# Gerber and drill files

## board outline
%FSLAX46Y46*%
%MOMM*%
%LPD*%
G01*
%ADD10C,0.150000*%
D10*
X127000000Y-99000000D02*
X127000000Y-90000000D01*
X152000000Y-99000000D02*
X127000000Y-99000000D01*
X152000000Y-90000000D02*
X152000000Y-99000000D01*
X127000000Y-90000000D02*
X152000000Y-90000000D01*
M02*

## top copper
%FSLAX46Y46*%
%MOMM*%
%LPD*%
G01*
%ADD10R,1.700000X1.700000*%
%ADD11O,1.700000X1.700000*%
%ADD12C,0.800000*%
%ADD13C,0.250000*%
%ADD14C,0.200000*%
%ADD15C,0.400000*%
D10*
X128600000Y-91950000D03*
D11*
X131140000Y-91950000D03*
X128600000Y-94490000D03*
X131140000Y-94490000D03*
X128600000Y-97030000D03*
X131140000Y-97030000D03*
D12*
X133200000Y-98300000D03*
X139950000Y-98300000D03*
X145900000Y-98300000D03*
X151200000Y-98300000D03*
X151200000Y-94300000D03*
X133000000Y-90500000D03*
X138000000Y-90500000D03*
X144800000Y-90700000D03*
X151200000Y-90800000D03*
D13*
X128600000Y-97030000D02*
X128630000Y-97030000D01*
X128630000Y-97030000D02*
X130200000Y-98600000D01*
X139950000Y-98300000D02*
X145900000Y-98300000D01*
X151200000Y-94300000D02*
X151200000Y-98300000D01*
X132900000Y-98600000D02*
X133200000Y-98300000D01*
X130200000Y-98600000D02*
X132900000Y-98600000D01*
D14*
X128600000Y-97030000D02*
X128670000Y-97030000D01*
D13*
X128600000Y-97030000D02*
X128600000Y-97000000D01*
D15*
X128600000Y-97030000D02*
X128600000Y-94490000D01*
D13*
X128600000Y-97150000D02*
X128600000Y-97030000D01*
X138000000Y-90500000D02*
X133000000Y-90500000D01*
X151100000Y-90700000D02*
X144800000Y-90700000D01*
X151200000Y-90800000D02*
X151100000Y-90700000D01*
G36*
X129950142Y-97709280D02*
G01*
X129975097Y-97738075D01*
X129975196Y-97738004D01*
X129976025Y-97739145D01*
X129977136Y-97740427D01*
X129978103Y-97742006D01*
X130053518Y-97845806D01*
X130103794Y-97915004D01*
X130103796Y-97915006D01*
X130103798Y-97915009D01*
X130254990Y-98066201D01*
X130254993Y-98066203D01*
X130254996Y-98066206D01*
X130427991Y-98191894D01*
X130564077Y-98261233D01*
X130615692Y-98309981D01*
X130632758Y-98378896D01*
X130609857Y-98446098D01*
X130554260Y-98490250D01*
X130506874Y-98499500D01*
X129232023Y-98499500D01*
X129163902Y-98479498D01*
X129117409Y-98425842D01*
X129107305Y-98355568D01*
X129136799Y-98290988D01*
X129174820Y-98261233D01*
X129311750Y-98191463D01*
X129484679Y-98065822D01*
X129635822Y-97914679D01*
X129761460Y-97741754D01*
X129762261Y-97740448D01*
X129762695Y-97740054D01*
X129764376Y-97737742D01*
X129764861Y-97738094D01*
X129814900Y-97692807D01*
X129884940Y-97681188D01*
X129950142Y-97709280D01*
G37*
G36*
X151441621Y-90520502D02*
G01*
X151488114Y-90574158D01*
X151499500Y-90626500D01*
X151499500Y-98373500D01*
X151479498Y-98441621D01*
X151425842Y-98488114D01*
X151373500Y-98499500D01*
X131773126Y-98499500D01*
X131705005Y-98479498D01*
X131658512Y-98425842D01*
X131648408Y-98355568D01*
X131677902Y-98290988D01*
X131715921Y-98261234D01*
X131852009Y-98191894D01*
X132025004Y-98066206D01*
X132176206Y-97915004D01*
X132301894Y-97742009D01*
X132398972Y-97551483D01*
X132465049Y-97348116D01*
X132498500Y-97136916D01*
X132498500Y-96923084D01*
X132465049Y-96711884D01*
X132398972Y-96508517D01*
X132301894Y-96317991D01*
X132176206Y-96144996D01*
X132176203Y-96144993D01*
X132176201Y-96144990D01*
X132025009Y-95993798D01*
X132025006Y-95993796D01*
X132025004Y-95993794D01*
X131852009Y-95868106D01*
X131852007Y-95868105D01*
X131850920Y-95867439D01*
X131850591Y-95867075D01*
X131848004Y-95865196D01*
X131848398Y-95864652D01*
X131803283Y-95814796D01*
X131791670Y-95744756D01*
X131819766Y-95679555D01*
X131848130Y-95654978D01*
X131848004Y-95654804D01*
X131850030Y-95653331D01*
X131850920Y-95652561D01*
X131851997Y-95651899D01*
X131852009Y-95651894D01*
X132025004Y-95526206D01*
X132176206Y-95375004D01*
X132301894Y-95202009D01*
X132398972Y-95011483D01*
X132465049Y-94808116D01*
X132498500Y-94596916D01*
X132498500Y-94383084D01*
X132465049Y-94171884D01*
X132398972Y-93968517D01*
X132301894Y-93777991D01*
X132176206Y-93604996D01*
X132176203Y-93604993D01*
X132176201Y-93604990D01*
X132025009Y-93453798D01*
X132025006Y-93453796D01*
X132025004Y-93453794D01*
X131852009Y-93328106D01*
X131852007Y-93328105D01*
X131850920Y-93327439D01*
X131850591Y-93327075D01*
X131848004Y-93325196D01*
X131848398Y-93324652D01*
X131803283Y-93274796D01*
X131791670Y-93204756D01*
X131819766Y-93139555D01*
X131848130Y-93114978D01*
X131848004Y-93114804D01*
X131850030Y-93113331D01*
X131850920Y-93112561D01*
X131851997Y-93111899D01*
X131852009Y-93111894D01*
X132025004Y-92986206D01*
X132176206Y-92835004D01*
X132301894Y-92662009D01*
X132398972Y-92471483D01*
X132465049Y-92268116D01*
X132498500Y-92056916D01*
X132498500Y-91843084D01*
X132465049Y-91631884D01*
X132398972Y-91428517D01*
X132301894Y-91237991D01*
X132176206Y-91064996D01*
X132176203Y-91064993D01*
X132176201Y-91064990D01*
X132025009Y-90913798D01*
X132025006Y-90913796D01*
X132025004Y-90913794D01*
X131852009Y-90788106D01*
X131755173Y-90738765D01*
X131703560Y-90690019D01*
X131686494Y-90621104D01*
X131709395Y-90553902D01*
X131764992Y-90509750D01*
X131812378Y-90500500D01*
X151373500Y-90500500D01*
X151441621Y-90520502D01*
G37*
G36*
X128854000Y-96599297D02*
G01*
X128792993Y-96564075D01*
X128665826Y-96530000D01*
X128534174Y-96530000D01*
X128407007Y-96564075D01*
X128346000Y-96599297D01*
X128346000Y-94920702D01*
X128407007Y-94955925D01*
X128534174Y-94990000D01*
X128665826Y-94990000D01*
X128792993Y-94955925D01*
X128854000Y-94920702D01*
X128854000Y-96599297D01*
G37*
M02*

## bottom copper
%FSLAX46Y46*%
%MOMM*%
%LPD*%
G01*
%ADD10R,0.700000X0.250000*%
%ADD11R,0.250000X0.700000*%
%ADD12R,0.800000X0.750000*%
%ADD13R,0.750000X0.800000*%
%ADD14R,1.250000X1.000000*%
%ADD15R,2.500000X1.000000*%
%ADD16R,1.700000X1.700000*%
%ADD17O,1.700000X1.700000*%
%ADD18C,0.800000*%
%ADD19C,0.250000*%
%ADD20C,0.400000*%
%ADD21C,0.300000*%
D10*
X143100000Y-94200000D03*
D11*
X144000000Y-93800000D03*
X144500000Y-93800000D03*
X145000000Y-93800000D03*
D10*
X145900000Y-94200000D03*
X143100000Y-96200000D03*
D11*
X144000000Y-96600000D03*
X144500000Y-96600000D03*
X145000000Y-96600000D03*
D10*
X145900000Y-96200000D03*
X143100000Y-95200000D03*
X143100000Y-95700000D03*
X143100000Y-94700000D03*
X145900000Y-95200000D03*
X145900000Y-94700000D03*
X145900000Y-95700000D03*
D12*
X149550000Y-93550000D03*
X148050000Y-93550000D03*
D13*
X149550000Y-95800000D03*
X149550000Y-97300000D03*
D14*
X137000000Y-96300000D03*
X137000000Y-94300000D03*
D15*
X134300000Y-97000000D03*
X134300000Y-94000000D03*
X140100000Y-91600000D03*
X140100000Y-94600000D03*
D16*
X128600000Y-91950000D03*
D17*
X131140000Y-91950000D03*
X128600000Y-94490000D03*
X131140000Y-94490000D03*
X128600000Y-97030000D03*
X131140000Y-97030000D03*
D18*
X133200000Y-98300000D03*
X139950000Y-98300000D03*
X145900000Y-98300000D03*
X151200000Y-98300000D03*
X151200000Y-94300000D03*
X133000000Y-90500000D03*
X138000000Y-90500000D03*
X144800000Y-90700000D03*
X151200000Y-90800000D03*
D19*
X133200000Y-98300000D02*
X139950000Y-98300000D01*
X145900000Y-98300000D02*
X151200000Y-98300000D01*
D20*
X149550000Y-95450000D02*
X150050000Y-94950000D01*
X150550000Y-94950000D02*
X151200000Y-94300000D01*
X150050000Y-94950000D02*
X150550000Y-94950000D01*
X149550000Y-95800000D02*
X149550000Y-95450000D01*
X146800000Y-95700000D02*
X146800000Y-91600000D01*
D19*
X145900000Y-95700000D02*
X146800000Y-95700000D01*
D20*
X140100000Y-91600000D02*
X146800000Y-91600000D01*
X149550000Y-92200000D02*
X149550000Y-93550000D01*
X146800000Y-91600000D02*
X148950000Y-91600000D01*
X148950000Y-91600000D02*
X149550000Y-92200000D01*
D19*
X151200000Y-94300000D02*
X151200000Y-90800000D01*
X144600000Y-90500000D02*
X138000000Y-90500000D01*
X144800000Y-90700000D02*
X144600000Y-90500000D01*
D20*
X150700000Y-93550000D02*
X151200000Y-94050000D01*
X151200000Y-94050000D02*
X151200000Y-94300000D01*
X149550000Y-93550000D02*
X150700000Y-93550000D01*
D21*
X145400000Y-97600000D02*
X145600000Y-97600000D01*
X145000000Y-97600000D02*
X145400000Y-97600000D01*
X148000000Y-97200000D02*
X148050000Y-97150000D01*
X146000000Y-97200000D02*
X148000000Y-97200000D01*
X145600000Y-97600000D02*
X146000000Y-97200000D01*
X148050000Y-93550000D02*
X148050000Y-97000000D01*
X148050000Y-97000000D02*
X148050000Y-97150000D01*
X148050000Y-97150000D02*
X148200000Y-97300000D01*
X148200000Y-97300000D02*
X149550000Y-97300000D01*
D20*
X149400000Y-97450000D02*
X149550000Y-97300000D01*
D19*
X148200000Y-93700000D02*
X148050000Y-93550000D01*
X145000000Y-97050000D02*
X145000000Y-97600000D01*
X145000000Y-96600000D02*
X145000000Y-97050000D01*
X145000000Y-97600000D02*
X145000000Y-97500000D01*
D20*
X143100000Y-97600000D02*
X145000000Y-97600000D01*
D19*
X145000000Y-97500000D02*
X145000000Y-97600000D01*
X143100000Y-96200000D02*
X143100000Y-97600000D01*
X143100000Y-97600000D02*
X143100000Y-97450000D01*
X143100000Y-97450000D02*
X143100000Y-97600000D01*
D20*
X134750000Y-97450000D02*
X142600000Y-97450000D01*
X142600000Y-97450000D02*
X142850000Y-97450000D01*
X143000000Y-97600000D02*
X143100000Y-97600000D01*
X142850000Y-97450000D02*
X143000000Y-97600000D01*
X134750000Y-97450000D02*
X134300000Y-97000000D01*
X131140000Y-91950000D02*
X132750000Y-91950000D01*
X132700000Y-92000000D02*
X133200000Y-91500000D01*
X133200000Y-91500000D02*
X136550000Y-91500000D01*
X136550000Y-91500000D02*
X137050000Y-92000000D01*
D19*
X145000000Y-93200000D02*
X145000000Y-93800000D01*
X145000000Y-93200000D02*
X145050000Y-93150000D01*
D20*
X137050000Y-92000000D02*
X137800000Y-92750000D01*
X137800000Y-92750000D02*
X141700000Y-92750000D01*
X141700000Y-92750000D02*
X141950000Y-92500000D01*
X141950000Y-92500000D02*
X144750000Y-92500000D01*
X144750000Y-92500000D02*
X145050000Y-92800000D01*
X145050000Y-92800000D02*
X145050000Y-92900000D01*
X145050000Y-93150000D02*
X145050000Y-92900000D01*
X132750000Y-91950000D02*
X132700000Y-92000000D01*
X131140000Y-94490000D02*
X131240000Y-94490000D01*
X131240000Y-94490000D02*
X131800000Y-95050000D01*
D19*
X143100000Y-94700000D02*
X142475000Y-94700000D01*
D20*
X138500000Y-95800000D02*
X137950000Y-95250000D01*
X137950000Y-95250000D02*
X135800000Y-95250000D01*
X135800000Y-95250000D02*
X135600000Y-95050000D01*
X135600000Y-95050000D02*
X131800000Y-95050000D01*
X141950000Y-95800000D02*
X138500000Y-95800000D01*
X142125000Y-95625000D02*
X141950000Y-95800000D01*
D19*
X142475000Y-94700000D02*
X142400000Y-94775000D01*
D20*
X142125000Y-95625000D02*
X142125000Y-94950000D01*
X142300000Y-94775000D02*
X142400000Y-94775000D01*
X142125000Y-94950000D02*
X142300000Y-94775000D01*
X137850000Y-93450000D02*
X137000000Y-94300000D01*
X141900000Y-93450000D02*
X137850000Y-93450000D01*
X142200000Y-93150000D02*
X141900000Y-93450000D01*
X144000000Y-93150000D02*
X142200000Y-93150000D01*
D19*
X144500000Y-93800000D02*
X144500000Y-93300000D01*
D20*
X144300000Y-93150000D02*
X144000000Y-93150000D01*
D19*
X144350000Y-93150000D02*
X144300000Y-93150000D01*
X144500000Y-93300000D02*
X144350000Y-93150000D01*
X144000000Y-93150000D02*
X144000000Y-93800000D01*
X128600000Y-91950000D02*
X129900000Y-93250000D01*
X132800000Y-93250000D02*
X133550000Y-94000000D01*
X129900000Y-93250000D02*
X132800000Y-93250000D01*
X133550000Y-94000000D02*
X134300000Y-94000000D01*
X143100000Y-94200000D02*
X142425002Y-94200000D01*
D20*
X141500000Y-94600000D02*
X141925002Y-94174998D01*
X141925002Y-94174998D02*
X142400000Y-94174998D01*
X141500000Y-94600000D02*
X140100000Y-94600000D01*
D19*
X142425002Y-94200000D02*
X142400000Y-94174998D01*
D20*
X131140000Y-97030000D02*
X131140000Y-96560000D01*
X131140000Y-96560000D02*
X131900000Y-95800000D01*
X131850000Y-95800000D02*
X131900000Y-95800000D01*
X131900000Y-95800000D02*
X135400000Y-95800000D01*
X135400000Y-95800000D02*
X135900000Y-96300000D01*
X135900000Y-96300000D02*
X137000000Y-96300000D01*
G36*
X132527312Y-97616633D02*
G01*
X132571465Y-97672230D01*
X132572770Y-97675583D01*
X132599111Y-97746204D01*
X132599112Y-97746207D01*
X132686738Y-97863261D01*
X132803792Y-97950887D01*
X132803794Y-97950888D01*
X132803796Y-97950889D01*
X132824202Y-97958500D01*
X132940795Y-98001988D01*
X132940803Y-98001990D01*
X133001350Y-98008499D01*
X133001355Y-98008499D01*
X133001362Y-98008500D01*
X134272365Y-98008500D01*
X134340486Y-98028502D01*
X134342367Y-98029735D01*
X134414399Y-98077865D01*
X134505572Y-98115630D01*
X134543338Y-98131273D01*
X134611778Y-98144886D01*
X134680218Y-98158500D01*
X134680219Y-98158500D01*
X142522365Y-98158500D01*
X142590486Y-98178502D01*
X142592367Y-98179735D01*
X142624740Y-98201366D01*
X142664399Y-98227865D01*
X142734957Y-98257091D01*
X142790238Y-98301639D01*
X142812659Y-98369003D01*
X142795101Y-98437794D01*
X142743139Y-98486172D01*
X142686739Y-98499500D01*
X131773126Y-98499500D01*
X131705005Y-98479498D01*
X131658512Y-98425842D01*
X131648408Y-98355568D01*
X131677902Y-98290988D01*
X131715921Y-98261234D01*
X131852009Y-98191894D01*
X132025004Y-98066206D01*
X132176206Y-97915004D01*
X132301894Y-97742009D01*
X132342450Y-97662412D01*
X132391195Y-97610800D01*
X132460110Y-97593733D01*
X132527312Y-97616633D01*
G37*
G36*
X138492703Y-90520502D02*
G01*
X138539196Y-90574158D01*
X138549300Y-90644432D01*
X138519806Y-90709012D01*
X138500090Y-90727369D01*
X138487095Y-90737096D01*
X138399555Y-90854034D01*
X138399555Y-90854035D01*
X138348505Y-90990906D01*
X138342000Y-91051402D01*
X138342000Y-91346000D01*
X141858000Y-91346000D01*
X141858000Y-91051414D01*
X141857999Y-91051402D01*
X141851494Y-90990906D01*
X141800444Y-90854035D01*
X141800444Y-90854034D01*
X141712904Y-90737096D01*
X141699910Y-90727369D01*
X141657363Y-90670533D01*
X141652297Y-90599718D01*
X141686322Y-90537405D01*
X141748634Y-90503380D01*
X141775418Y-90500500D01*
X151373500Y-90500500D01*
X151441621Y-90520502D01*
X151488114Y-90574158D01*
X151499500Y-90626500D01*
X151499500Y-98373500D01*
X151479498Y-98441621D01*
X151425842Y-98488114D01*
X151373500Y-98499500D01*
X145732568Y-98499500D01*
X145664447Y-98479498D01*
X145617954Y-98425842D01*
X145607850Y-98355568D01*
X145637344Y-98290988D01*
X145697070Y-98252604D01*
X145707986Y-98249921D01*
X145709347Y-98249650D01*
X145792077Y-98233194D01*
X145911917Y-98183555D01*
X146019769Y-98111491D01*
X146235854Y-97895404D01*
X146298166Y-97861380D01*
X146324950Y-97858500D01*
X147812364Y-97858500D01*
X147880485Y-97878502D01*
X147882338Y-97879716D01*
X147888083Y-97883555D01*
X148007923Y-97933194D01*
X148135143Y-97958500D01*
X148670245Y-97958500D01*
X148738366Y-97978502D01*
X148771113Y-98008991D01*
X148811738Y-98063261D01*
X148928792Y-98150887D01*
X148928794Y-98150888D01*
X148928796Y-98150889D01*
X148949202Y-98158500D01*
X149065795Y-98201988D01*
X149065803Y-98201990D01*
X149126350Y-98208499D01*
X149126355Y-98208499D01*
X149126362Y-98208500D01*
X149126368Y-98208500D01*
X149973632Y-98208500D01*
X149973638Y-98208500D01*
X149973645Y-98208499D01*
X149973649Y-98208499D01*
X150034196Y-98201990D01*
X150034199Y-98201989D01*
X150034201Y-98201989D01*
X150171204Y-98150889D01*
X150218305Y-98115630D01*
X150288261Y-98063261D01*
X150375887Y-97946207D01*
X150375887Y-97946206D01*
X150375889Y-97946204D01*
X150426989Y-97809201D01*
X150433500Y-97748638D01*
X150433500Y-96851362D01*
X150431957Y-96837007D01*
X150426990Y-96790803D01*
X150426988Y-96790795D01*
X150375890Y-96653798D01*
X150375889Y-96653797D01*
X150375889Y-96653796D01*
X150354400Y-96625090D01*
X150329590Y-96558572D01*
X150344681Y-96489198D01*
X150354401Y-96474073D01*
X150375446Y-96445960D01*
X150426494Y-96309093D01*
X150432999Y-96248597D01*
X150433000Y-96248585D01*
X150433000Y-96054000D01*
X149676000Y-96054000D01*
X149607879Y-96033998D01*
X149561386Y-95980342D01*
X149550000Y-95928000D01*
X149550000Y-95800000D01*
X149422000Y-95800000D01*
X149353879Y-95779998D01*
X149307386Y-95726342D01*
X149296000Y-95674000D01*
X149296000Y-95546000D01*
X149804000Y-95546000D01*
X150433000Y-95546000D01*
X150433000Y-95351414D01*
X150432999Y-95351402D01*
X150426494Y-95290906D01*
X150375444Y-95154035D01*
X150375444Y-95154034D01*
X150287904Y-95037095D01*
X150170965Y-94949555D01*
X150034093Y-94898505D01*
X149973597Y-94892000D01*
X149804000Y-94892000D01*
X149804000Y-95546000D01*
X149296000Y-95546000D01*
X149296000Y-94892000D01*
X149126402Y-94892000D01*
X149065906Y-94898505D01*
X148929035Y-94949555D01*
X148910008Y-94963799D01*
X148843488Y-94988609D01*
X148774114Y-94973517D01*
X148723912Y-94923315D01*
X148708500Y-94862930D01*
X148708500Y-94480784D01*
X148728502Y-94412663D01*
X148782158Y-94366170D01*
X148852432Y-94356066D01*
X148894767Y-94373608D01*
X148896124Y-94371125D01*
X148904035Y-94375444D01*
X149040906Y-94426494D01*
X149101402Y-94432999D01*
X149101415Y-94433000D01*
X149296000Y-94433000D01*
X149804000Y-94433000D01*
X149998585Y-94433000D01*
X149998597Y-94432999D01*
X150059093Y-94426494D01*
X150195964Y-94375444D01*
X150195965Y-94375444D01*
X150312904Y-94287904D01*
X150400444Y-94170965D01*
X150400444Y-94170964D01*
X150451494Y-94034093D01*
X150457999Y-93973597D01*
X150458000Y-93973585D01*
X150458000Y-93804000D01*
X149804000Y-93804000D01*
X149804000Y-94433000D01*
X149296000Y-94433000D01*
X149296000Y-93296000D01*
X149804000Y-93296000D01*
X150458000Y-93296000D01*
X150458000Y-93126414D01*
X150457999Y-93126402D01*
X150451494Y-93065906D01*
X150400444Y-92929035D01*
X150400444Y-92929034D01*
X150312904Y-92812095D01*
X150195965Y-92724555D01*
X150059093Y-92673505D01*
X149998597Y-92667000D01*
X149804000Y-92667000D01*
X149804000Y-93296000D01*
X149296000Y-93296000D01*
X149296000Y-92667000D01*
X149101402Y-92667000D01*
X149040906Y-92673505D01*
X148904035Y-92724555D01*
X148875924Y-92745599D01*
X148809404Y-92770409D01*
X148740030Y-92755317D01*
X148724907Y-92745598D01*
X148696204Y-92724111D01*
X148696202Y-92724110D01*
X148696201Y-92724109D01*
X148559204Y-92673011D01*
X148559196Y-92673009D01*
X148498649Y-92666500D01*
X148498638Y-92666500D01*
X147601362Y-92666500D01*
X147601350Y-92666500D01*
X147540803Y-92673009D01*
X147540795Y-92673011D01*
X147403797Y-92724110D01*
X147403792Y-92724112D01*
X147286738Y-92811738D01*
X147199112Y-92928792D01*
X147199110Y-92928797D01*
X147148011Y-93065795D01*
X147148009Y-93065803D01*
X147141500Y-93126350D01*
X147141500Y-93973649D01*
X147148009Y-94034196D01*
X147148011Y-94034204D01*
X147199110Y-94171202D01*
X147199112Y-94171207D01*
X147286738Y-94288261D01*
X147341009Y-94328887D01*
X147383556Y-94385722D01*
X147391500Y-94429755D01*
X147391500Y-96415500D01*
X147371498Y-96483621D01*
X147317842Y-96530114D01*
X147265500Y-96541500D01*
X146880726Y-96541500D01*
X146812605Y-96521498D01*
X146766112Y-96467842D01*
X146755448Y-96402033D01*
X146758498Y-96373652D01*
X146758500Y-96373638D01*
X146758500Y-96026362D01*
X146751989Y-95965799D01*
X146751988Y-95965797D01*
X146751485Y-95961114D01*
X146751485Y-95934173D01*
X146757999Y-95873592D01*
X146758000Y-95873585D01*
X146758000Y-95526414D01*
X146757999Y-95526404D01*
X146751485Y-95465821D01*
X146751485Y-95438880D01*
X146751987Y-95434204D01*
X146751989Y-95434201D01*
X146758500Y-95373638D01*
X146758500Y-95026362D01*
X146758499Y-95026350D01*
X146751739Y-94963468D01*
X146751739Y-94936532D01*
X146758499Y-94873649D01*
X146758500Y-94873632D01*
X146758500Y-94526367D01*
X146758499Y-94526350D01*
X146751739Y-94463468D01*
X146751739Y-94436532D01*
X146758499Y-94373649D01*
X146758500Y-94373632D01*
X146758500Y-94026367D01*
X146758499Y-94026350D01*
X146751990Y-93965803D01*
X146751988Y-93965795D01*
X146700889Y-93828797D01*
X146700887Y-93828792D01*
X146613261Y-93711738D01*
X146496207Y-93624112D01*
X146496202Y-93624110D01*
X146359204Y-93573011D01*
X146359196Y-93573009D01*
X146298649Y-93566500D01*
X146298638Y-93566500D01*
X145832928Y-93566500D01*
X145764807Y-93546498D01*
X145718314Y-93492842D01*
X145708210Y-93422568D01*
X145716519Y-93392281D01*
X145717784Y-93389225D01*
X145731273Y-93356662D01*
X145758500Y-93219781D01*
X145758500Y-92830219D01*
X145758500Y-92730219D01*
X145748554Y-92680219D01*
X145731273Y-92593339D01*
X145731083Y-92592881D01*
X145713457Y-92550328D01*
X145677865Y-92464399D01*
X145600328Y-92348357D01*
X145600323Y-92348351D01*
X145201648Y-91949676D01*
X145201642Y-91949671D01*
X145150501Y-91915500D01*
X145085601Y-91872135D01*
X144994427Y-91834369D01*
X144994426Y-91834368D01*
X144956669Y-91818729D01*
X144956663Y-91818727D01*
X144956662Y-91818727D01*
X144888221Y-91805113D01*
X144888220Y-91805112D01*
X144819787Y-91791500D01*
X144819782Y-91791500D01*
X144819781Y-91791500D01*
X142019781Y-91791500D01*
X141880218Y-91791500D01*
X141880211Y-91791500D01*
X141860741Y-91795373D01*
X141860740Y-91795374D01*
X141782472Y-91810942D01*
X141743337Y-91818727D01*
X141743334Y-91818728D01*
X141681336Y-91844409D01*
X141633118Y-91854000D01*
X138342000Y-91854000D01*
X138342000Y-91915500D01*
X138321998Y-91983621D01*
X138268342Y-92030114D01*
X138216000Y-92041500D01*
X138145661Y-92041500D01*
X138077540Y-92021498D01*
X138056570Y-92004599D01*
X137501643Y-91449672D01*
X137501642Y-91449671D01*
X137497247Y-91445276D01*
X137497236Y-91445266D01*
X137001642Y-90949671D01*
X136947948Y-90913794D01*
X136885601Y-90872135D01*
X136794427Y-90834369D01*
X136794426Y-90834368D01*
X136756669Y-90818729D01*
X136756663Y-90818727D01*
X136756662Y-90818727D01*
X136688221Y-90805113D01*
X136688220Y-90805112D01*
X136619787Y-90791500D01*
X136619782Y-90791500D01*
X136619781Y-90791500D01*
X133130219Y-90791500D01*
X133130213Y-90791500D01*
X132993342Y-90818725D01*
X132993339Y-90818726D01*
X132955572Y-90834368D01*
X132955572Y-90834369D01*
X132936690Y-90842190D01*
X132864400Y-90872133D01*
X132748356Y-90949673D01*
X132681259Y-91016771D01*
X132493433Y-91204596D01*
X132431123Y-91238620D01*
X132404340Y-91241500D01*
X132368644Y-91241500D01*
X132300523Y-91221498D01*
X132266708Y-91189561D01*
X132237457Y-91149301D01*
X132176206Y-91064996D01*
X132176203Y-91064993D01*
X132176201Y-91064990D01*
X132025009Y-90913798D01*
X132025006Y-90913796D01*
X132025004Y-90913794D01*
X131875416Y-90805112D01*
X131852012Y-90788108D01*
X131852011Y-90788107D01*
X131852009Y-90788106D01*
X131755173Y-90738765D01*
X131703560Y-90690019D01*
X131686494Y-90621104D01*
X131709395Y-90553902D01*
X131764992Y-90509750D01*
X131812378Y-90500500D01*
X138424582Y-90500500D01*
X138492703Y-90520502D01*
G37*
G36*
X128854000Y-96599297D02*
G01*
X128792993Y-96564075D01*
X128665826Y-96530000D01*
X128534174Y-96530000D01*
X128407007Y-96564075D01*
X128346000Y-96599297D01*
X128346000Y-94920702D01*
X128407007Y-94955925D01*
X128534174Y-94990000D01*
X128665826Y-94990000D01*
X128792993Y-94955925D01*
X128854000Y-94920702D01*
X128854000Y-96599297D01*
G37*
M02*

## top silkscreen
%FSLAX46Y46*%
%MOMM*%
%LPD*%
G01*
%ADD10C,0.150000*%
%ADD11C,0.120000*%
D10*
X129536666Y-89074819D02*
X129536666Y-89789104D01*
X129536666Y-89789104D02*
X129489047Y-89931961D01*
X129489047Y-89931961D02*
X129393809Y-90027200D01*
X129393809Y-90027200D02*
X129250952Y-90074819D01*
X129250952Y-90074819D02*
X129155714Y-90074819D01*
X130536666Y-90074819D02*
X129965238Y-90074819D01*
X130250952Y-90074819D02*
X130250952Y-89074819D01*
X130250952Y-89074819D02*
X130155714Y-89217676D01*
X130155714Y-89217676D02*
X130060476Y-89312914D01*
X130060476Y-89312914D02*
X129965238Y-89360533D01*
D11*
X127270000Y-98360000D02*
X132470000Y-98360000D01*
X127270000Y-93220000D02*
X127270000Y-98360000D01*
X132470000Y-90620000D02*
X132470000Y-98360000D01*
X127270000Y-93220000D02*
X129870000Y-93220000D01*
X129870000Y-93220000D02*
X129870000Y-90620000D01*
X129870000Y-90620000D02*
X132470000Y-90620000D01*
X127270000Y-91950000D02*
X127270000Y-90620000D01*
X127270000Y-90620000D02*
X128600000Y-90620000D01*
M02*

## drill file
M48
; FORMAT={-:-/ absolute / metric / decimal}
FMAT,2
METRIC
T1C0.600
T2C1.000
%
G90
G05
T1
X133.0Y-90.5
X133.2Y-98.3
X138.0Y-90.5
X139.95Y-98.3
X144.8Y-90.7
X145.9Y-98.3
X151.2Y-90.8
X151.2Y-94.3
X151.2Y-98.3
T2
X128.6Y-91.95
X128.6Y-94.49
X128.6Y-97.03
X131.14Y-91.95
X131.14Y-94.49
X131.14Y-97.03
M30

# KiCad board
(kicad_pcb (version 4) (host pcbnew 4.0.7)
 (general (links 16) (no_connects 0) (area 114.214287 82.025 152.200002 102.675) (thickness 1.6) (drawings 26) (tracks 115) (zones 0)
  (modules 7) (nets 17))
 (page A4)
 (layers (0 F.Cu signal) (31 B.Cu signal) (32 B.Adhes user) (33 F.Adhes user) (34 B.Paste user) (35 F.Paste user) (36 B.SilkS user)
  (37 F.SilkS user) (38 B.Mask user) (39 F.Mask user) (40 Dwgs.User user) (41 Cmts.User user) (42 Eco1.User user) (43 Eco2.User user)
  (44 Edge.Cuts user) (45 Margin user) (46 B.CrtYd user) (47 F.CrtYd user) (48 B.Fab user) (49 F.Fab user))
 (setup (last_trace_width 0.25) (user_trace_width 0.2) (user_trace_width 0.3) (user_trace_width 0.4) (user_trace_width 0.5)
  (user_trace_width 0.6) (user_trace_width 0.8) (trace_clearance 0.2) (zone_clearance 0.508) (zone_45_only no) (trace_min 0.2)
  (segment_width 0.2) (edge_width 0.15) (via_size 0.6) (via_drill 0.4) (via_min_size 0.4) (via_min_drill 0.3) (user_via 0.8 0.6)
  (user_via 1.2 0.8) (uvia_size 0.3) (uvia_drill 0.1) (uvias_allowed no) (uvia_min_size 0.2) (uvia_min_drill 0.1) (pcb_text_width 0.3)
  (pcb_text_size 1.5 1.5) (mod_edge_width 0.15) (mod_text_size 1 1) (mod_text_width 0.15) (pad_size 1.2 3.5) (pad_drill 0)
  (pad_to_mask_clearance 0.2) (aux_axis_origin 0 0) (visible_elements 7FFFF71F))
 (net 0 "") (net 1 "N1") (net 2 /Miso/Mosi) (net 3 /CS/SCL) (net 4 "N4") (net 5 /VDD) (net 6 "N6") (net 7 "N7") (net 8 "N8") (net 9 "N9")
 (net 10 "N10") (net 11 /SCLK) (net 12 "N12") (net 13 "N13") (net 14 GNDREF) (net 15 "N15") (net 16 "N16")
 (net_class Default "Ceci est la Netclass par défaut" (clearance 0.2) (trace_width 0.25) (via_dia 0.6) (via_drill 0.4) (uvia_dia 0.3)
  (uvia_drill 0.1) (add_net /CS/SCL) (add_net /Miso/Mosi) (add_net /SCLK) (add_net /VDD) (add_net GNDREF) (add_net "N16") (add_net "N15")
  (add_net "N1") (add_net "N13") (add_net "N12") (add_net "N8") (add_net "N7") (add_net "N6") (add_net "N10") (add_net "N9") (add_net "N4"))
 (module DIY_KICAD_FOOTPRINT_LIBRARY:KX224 (layer B.Cu) (at 144.5 95.2)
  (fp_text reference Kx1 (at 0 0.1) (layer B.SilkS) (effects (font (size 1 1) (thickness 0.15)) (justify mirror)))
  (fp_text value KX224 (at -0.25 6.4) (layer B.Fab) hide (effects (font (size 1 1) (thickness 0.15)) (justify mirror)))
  (pad 5 smd rect (at -1.4 -1 270) (size 0.25 0.7) (layers B.Cu B.Paste B.Mask) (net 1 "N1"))
  (pad 6 smd rect (at -0.5 -1.4) (size 0.25 0.7) (layers B.Cu B.Paste B.Mask) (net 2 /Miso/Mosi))
  (pad 7 smd rect (at 0 -1.4) (size 0.25 0.7) (layers B.Cu B.Paste B.Mask) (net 2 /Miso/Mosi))
  (pad 8 smd rect (at 0.5 -1.4) (size 0.25 0.7) (layers B.Cu B.Paste B.Mask) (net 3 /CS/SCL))
  (pad 9 smd rect (at 1.4 -1 270) (size 0.25 0.7) (layers B.Cu B.Paste B.Mask) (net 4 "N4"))
  (pad 1 smd rect (at -1.4 1 270) (size 0.25 0.7) (layers B.Cu B.Paste B.Mask) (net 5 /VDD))
  (pad 16 smd rect (at -0.5 1.4) (size 0.25 0.7) (layers B.Cu B.Paste B.Mask) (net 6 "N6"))
  (pad 15 smd rect (at 0 1.4) (size 0.25 0.7) (layers B.Cu B.Paste B.Mask) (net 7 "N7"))
  (pad 14 smd rect (at 0.5 1.4) (size 0.25 0.7) (layers B.Cu B.Paste B.Mask) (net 5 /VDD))
  (pad 13 smd rect (at 1.4 1 270) (size 0.25 0.7) (layers B.Cu B.Paste B.Mask) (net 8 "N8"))
  (pad 3 smd rect (at -1.4 0 270) (size 0.25 0.7) (layers B.Cu B.Paste B.Mask) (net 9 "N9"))
  (pad 2 smd rect (at -1.4 0.5 270) (size 0.25 0.7) (layers B.Cu B.Paste B.Mask) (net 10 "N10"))
  (pad 4 smd rect (at -1.4 -0.5 270) (size 0.25 0.7) (layers B.Cu B.Paste B.Mask) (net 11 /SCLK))
  (pad 11 smd rect (at 1.4 0 270) (size 0.25 0.7) (layers B.Cu B.Paste B.Mask) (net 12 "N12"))
  (pad 10 smd rect (at 1.4 -0.5 270) (size 0.25 0.7) (layers B.Cu B.Paste B.Mask) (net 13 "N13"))
  (pad 12 smd rect (at 1.4 0.5 270) (size 0.25 0.7) (layers B.Cu B.Paste B.Mask) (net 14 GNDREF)))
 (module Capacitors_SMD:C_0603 (layer B.Cu) (at 148.8 93.55)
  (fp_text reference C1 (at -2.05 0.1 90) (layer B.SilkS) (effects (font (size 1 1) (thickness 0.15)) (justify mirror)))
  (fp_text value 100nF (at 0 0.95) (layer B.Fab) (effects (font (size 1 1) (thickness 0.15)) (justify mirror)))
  (pad 2 smd rect (at 0.75 0) (size 0.8 0.75) (layers B.Cu B.Paste B.Mask) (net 14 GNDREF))
  (pad 1 smd rect (at -0.75 0) (size 0.8 0.75) (layers B.Cu B.Paste B.Mask) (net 5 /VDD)))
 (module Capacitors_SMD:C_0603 (layer B.Cu) (at 149.55 96.55 90)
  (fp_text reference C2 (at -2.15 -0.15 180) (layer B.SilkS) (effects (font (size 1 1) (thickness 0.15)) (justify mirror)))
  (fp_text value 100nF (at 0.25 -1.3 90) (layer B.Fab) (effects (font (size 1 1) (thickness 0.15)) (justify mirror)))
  (pad 2 smd rect (at 0.75 0 90) (size 0.8 0.75) (layers B.Cu B.Paste B.Mask) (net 14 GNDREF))
  (pad 1 smd rect (at -0.75 0 90) (size 0.8 0.75) (layers B.Cu B.Paste B.Mask) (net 5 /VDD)))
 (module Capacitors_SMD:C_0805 (layer B.Cu) (at 137 95.3 90)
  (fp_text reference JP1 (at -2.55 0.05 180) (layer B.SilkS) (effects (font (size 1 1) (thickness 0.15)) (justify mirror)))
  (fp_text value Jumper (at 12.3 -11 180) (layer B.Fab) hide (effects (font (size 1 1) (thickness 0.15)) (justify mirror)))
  (pad 1 smd rect (at -1 0 90) (size 1 1.25) (layers B.Cu B.Paste B.Mask) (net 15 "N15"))
  (pad 2 smd rect (at 1 0 90) (size 1 1.25) (layers B.Cu B.Paste B.Mask) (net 2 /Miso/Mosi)))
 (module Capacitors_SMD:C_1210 (layer B.Cu) (at 134.3 95.5 90)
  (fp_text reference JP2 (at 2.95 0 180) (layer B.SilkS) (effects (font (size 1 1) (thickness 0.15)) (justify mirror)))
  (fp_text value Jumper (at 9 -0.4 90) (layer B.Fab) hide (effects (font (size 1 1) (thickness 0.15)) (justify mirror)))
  (pad 1 smd rect (at -1.5 0 90) (size 1 2.5) (layers B.Cu B.Paste B.Mask) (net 5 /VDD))
  (pad 2 smd rect (at 1.5 0 90) (size 1 2.5) (layers B.Cu B.Paste B.Mask) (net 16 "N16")))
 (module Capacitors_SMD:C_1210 (layer B.Cu) (at 140.1 93.1 270)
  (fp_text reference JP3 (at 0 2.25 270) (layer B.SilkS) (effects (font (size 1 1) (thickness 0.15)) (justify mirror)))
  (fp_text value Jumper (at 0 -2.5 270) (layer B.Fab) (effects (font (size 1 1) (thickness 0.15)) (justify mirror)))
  (pad 1 smd rect (at -1.5 0 270) (size 1 2.5) (layers B.Cu B.Paste B.Mask) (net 14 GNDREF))
  (pad 2 smd rect (at 1.5 0 270) (size 1 2.5) (layers B.Cu B.Paste B.Mask) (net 1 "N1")))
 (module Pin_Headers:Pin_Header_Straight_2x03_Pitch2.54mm (layer F.Cu) (at 128.6 91.95)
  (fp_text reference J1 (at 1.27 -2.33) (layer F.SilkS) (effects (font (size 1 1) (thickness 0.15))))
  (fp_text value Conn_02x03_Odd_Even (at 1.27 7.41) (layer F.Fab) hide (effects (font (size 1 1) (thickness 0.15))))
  (fp_line (start -1.33 6.41) (end 3.87 6.41) (layer F.SilkS) (width 0.12))
  (fp_line (start -1.33 1.27) (end -1.33 6.41) (layer F.SilkS) (width 0.12))
  (fp_line (start 3.87 -1.33) (end 3.87 6.41) (layer F.SilkS) (width 0.12))
  (fp_line (start -1.33 1.27) (end 1.27 1.27) (layer F.SilkS) (width 0.12))
  (fp_line (start 1.27 1.27) (end 1.27 -1.33) (layer F.SilkS) (width 0.12))
  (fp_line (start 1.27 -1.33) (end 3.87 -1.33) (layer F.SilkS) (width 0.12))
  (fp_line (start -1.33 0) (end -1.33 -1.33) (layer F.SilkS) (width 0.12))
  (fp_line (start -1.33 -1.33) (end 0 -1.33) (layer F.SilkS) (width 0.12))
  (pad 1 thru_hole rect (at 0 0) (size 1.7 1.7) (drill 1) (layers *.Cu *.Mask) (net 16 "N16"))
  (pad 2 thru_hole oval (at 2.54 0) (size 1.7 1.7) (drill 1) (layers *.Cu *.Mask) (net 3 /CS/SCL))
  (pad 3 thru_hole oval (at 0 2.54) (size 1.7 1.7) (drill 1) (layers *.Cu *.Mask) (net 14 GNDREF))
  (pad 4 thru_hole oval (at 2.54 2.54) (size 1.7 1.7) (drill 1) (layers *.Cu *.Mask) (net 11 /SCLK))
  (pad 5 thru_hole oval (at 0 5.08) (size 1.7 1.7) (drill 1) (layers *.Cu *.Mask) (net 14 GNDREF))
  (pad 6 thru_hole oval (at 2.54 5.08) (size 1.7 1.7) (drill 1) (layers *.Cu *.Mask) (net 15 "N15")))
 (gr_line (start 127 99) (end 127 90) (angle 90) (layer Edge.Cuts) (width 0.15))
 (gr_line (start 152 99) (end 127 99) (angle 90) (layer Edge.Cuts) (width 0.15))
 (gr_line (start 152 90) (end 152 99) (angle 90) (layer Edge.Cuts) (width 0.15))
 (gr_line (start 127 90) (end 152 90) (angle 90) (layer Edge.Cuts) (width 0.15))
 (segment (start 128.6 97.03) (end 128.63 97.03) (width 0.25) (layer F.Cu) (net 14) (status C00000))
 (segment (start 128.63 97.03) (end 130.2 98.6) (width 0.25) (layer F.Cu) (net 14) (status 400000))
 (via (at 133.2 98.3) (size 0.8) (drill 0.6) (layers F.Cu B.Cu) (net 14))
 (segment (start 133.2 98.3) (end 139.95 98.3) (width 0.25) (layer B.Cu) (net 14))
 (via (at 139.95 98.3) (size 0.8) (drill 0.6) (layers F.Cu B.Cu) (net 14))
 (segment (start 139.95 98.3) (end 145.9 98.3) (width 0.25) (layer F.Cu) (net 14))
 (via (at 145.9 98.3) (size 0.8) (drill 0.6) (layers F.Cu B.Cu) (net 14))
 (segment (start 145.9 98.3) (end 151.2 98.3) (width 0.25) (layer B.Cu) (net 14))
 (via (at 151.2 98.3) (size 0.8) (drill 0.6) (layers F.Cu B.Cu) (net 14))
 (segment (start 151.2 94.3) (end 151.2 98.3) (width 0.25) (layer F.Cu) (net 14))
 (via (at 151.2 94.3) (size 0.8) (drill 0.6) (layers F.Cu B.Cu) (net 14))
 (segment (start 132.9 98.6) (end 133.2 98.3) (width 0.25) (layer F.Cu) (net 14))
 (segment (start 130.2 98.6) (end 132.9 98.6) (width 0.25) (layer F.Cu) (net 14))
 (segment (start 128.6 97.03) (end 128.67 97.03) (width 0.2) (layer F.Cu) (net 14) (status C00000))
 (segment (start 128.6 97.03) (end 128.6 97) (width 0.25) (layer F.Cu) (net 14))
 (segment (start 149.55 95.45) (end 150.05 94.95) (width 0.4) (layer B.Cu) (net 14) (status 10))
 (segment (start 150.55 94.95) (end 151.2 94.3) (width 0.4) (layer B.Cu) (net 14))
 (segment (start 150.05 94.95) (end 150.55 94.95) (width 0.4) (layer B.Cu) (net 14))
 (segment (start 149.55 95.8) (end 149.55 95.45) (width 0.4) (layer B.Cu) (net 14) (status 30))
 (segment (start 146.8 95.7) (end 146.8 91.6) (width 0.4) (layer B.Cu) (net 14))
 (segment (start 145.9 95.7) (end 146.8 95.7) (width 0.25) (layer B.Cu) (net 14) (status 10))
 (segment (start 140.1 91.6) (end 146.8 91.6) (width 0.4) (layer B.Cu) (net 14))
 (segment (start 149.55 92.2) (end 149.55 93.55) (width 0.4) (layer B.Cu) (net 14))
 (segment (start 146.8 91.6) (end 148.95 91.6) (width 0.4) (layer B.Cu) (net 14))
 (segment (start 148.95 91.6) (end 149.55 92.2) (width 0.4) (layer B.Cu) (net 14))
 (segment (start 128.6 97.03) (end 128.6 94.49) (width 0.4) (layer F.Cu) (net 14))
 (segment (start 128.6 97.15) (end 128.6 97.03) (width 0.25) (layer F.Cu) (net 14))
 (segment (start 151.2 94.3) (end 151.2 90.8) (width 0.25) (layer B.Cu) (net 14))
 (via (at 133 90.5) (size 0.8) (drill 0.6) (layers F.Cu B.Cu) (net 14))
 (segment (start 138 90.5) (end 133 90.5) (width 0.25) (layer F.Cu) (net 14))
 (via (at 138 90.5) (size 0.8) (drill 0.6) (layers F.Cu B.Cu) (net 14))
 (segment (start 144.6 90.5) (end 138 90.5) (width 0.25) (layer B.Cu) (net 14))
 (segment (start 144.8 90.7) (end 144.6 90.5) (width 0.25) (layer B.Cu) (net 14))
 (via (at 144.8 90.7) (size 0.8) (drill 0.6) (layers F.Cu B.Cu) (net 14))
 (segment (start 151.1 90.7) (end 144.8 90.7) (width 0.25) (layer F.Cu) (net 14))
 (segment (start 151.2 90.8) (end 151.1 90.7) (width 0.25) (layer F.Cu) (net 14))
 (via (at 151.2 90.8) (size 0.8) (drill 0.6) (layers F.Cu B.Cu) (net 14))
 (segment (start 150.7 93.55) (end 151.2 94.05) (width 0.4) (layer B.Cu) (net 14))
 (segment (start 151.2 94.05) (end 151.2 94.3) (width 0.4) (layer B.Cu) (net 14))
 (segment (start 149.55 93.55) (end 150.7 93.55) (width 0.4) (layer B.Cu) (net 14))
 (segment (start 145.4 97.6) (end 145.6 97.6) (width 0.3) (layer B.Cu) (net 5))
 (segment (start 145 97.6) (end 145.4 97.6) (width 0.3) (layer B.Cu) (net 5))
 (segment (start 148 97.2) (end 148.05 97.15) (width 0.3) (layer B.Cu) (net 5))
 (segment (start 146 97.2) (end 148 97.2) (width 0.3) (layer B.Cu) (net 5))
 (segment (start 145.6 97.6) (end 146 97.2) (width 0.3) (layer B.Cu) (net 5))
 (segment (start 148.05 93.55) (end 148.05 97) (width 0.3) (layer B.Cu) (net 5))
 (segment (start 148.05 97) (end 148.05 97.15) (width 0.3) (layer B.Cu) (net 5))
 (segment (start 148.05 97.15) (end 148.2 97.3) (width 0.3) (layer B.Cu) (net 5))
 (segment (start 148.2 97.3) (end 149.55 97.3) (width 0.3) (layer B.Cu) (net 5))
 (segment (start 149.4 97.45) (end 149.55 97.3) (width 0.4) (layer B.Cu) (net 5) (status 30))
 (segment (start 148.2 93.7) (end 148.05 93.55) (width 0.25) (layer B.Cu) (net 5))
 (segment (start 145 97.05) (end 145 97.6) (width 0.25) (layer B.Cu) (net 5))
 (segment (start 145 96.6) (end 145 97.05) (width 0.25) (layer B.Cu) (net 5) (status 10))
 (segment (start 145 97.6) (end 145 97.5) (width 0.25) (layer B.Cu) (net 5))
 (segment (start 143.1 97.6) (end 145 97.6) (width 0.4) (layer B.Cu) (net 5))
 (segment (start 145 97.5) (end 145 97.6) (width 0.25) (layer B.Cu) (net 5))
 (segment (start 143.1 96.2) (end 143.1 97.6) (width 0.25) (layer B.Cu) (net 5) (status 10))
 (segment (start 143.1 97.6) (end 143.1 97.45) (width 0.25) (layer B.Cu) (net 5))
 (segment (start 143.1 97.45) (end 143.1 97.6) (width 0.25) (layer B.Cu) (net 5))
 (segment (start 134.75 97.45) (end 142.6 97.45) (width 0.4) (layer B.Cu) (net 5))
 (segment (start 142.6 97.45) (end 142.85 97.45) (width 0.4) (layer B.Cu) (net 5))
 (segment (start 143 97.6) (end 143.1 97.6) (width 0.4) (layer B.Cu) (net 5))
 (segment (start 142.85 97.45) (end 143 97.6) (width 0.4) (layer B.Cu) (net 5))
 (segment (start 134.75 97.45) (end 134.3 97) (width 0.4) (layer B.Cu) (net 5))
 (segment (start 131.14 91.95) (end 132.75 91.95) (width 0.4) (layer B.Cu) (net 3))
 (segment (start 132.7 92) (end 133.2 91.5) (width 0.4) (layer B.Cu) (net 3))
 (segment (start 133.2 91.5) (end 136.55 91.5) (width 0.4) (layer B.Cu) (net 3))
 (segment (start 136.55 91.5) (end 137.05 92) (width 0.4) (layer B.Cu) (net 3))
 (segment (start 145 93.2) (end 145 93.8) (width 0.25) (layer B.Cu) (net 3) (status 20))
 (segment (start 145 93.2) (end 145.05 93.15) (width 0.25) (layer B.Cu) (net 3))
 (segment (start 137.05 92) (end 137.8 92.75) (width 0.4) (layer B.Cu) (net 3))
 (segment (start 137.8 92.75) (end 141.7 92.75) (width 0.4) (layer B.Cu) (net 3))
 (segment (start 141.7 92.75) (end 141.95 92.5) (width 0.4) (layer B.Cu) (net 3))
 (segment (start 141.95 92.5) (end 144.75 92.5) (width 0.4) (layer B.Cu) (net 3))
 (segment (start 144.75 92.5) (end 145.05 92.8) (width 0.4) (layer B.Cu) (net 3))
 (segment (start 145.05 92.8) (end 145.05 92.9) (width 0.4) (layer B.Cu) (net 3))
 (segment (start 145.05 93.15) (end 145.05 92.9) (width 0.4) (layer B.Cu) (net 3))
 (segment (start 132.75 91.95) (end 132.7 92) (width 0.4) (layer B.Cu) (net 3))
 (segment (start 131.14 94.49) (end 131.24 94.49) (width 0.4) (layer B.Cu) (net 11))
 (segment (start 131.24 94.49) (end 131.8 95.05) (width 0.4) (layer B.Cu) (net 11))
 (segment (start 143.1 94.7) (end 142.475 94.7) (width 0.25) (layer B.Cu) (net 11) (status 10))
 (segment (start 138.5 95.8) (end 137.95 95.25) (width 0.4) (layer B.Cu) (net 11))
 (segment (start 137.95 95.25) (end 135.8 95.25) (width 0.4) (layer B.Cu) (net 11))
 (segment (start 135.8 95.25) (end 135.6 95.05) (width 0.4) (layer B.Cu) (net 11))
 (segment (start 135.6 95.05) (end 131.8 95.05) (width 0.4) (layer B.Cu) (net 11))
 (segment (start 141.95 95.8) (end 138.5 95.8) (width 0.4) (layer B.Cu) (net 11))
 (segment (start 142.125 95.625) (end 141.95 95.8) (width 0.4) (layer B.Cu) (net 11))
 (segment (start 142.475 94.7) (end 142.4 94.775) (width 0.25) (layer B.Cu) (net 11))
 (segment (start 142.125 95.625) (end 142.125 94.95) (width 0.4) (layer B.Cu) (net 11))
 (segment (start 142.3 94.775) (end 142.4 94.775) (width 0.4) (layer B.Cu) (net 11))
 (segment (start 142.125 94.95) (end 142.3 94.775) (width 0.4) (layer B.Cu) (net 11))
 (segment (start 137.85 93.45) (end 137 94.3) (width 0.4) (layer B.Cu) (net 2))
 (segment (start 141.9 93.45) (end 137.85 93.45) (width 0.4) (layer B.Cu) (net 2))
 (segment (start 142.2 93.15) (end 141.9 93.45) (width 0.4) (layer B.Cu) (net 2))
 (segment (start 144 93.15) (end 142.2 93.15) (width 0.4) (layer B.Cu) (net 2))
 (segment (start 144.5 93.8) (end 144.5 93.3) (width 0.25) (layer B.Cu) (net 2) (status 10))
 (segment (start 144.3 93.15) (end 144 93.15) (width 0.4) (layer B.Cu) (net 2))
 (segment (start 144.35 93.15) (end 144.3 93.15) (width 0.25) (layer B.Cu) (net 2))
 (segment (start 144.5 93.3) (end 144.35 93.15) (width 0.25) (layer B.Cu) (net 2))
 (segment (start 144 93.15) (end 144 93.8) (width 0.25) (layer B.Cu) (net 2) (status 20))
 (segment (start 128.6 91.95) (end 129.9 93.25) (width 0.25) (layer B.Cu) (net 16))
 (segment (start 132.8 93.25) (end 133.55 94) (width 0.25) (layer B.Cu) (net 16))
 (segment (start 129.9 93.25) (end 132.8 93.25) (width 0.25) (layer B.Cu) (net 16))
 (segment (start 133.55 94) (end 134.3 94) (width 0.25) (layer B.Cu) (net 16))
 (segment (start 143.1 94.2) (end 142.425002 94.2) (width 0.25) (layer B.Cu) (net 1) (status 10))
 (segment (start 141.5 94.6) (end 141.925002 94.174998) (width 0.4) (layer B.Cu) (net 1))
 (segment (start 141.925002 94.174998) (end 142.4 94.174998) (width 0.4) (layer B.Cu) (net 1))
 (segment (start 141.5 94.6) (end 140.1 94.6) (width 0.4) (layer B.Cu) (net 1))
 (segment (start 142.425002 94.2) (end 142.4 94.174998) (width 0.25) (layer B.Cu) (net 1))
 (segment (start 131.14 97.03) (end 131.14 96.56) (width 0.4) (layer B.Cu) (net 15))
 (segment (start 131.14 96.56) (end 131.9 95.8) (width 0.4) (layer B.Cu) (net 15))
 (segment (start 131.85 95.8) (end 131.9 95.8) (width 0.4) (layer B.Cu) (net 15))
 (segment (start 131.9 95.8) (end 135.4 95.8) (width 0.4) (layer B.Cu) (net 15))
 (segment (start 135.4 95.8) (end 135.9 96.3) (width 0.4) (layer B.Cu) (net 15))
 (segment (start 135.9 96.3) (end 137 96.3) (width 0.4) (layer B.Cu) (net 15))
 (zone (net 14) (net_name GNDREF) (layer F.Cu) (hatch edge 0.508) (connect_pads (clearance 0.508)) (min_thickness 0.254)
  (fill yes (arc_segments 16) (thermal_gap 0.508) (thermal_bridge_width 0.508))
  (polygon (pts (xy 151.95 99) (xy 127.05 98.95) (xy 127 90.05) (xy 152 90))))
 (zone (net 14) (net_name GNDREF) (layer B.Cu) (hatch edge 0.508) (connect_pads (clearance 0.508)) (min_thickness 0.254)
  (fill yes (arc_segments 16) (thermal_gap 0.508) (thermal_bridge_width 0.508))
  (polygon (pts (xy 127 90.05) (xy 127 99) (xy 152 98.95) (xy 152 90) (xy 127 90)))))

